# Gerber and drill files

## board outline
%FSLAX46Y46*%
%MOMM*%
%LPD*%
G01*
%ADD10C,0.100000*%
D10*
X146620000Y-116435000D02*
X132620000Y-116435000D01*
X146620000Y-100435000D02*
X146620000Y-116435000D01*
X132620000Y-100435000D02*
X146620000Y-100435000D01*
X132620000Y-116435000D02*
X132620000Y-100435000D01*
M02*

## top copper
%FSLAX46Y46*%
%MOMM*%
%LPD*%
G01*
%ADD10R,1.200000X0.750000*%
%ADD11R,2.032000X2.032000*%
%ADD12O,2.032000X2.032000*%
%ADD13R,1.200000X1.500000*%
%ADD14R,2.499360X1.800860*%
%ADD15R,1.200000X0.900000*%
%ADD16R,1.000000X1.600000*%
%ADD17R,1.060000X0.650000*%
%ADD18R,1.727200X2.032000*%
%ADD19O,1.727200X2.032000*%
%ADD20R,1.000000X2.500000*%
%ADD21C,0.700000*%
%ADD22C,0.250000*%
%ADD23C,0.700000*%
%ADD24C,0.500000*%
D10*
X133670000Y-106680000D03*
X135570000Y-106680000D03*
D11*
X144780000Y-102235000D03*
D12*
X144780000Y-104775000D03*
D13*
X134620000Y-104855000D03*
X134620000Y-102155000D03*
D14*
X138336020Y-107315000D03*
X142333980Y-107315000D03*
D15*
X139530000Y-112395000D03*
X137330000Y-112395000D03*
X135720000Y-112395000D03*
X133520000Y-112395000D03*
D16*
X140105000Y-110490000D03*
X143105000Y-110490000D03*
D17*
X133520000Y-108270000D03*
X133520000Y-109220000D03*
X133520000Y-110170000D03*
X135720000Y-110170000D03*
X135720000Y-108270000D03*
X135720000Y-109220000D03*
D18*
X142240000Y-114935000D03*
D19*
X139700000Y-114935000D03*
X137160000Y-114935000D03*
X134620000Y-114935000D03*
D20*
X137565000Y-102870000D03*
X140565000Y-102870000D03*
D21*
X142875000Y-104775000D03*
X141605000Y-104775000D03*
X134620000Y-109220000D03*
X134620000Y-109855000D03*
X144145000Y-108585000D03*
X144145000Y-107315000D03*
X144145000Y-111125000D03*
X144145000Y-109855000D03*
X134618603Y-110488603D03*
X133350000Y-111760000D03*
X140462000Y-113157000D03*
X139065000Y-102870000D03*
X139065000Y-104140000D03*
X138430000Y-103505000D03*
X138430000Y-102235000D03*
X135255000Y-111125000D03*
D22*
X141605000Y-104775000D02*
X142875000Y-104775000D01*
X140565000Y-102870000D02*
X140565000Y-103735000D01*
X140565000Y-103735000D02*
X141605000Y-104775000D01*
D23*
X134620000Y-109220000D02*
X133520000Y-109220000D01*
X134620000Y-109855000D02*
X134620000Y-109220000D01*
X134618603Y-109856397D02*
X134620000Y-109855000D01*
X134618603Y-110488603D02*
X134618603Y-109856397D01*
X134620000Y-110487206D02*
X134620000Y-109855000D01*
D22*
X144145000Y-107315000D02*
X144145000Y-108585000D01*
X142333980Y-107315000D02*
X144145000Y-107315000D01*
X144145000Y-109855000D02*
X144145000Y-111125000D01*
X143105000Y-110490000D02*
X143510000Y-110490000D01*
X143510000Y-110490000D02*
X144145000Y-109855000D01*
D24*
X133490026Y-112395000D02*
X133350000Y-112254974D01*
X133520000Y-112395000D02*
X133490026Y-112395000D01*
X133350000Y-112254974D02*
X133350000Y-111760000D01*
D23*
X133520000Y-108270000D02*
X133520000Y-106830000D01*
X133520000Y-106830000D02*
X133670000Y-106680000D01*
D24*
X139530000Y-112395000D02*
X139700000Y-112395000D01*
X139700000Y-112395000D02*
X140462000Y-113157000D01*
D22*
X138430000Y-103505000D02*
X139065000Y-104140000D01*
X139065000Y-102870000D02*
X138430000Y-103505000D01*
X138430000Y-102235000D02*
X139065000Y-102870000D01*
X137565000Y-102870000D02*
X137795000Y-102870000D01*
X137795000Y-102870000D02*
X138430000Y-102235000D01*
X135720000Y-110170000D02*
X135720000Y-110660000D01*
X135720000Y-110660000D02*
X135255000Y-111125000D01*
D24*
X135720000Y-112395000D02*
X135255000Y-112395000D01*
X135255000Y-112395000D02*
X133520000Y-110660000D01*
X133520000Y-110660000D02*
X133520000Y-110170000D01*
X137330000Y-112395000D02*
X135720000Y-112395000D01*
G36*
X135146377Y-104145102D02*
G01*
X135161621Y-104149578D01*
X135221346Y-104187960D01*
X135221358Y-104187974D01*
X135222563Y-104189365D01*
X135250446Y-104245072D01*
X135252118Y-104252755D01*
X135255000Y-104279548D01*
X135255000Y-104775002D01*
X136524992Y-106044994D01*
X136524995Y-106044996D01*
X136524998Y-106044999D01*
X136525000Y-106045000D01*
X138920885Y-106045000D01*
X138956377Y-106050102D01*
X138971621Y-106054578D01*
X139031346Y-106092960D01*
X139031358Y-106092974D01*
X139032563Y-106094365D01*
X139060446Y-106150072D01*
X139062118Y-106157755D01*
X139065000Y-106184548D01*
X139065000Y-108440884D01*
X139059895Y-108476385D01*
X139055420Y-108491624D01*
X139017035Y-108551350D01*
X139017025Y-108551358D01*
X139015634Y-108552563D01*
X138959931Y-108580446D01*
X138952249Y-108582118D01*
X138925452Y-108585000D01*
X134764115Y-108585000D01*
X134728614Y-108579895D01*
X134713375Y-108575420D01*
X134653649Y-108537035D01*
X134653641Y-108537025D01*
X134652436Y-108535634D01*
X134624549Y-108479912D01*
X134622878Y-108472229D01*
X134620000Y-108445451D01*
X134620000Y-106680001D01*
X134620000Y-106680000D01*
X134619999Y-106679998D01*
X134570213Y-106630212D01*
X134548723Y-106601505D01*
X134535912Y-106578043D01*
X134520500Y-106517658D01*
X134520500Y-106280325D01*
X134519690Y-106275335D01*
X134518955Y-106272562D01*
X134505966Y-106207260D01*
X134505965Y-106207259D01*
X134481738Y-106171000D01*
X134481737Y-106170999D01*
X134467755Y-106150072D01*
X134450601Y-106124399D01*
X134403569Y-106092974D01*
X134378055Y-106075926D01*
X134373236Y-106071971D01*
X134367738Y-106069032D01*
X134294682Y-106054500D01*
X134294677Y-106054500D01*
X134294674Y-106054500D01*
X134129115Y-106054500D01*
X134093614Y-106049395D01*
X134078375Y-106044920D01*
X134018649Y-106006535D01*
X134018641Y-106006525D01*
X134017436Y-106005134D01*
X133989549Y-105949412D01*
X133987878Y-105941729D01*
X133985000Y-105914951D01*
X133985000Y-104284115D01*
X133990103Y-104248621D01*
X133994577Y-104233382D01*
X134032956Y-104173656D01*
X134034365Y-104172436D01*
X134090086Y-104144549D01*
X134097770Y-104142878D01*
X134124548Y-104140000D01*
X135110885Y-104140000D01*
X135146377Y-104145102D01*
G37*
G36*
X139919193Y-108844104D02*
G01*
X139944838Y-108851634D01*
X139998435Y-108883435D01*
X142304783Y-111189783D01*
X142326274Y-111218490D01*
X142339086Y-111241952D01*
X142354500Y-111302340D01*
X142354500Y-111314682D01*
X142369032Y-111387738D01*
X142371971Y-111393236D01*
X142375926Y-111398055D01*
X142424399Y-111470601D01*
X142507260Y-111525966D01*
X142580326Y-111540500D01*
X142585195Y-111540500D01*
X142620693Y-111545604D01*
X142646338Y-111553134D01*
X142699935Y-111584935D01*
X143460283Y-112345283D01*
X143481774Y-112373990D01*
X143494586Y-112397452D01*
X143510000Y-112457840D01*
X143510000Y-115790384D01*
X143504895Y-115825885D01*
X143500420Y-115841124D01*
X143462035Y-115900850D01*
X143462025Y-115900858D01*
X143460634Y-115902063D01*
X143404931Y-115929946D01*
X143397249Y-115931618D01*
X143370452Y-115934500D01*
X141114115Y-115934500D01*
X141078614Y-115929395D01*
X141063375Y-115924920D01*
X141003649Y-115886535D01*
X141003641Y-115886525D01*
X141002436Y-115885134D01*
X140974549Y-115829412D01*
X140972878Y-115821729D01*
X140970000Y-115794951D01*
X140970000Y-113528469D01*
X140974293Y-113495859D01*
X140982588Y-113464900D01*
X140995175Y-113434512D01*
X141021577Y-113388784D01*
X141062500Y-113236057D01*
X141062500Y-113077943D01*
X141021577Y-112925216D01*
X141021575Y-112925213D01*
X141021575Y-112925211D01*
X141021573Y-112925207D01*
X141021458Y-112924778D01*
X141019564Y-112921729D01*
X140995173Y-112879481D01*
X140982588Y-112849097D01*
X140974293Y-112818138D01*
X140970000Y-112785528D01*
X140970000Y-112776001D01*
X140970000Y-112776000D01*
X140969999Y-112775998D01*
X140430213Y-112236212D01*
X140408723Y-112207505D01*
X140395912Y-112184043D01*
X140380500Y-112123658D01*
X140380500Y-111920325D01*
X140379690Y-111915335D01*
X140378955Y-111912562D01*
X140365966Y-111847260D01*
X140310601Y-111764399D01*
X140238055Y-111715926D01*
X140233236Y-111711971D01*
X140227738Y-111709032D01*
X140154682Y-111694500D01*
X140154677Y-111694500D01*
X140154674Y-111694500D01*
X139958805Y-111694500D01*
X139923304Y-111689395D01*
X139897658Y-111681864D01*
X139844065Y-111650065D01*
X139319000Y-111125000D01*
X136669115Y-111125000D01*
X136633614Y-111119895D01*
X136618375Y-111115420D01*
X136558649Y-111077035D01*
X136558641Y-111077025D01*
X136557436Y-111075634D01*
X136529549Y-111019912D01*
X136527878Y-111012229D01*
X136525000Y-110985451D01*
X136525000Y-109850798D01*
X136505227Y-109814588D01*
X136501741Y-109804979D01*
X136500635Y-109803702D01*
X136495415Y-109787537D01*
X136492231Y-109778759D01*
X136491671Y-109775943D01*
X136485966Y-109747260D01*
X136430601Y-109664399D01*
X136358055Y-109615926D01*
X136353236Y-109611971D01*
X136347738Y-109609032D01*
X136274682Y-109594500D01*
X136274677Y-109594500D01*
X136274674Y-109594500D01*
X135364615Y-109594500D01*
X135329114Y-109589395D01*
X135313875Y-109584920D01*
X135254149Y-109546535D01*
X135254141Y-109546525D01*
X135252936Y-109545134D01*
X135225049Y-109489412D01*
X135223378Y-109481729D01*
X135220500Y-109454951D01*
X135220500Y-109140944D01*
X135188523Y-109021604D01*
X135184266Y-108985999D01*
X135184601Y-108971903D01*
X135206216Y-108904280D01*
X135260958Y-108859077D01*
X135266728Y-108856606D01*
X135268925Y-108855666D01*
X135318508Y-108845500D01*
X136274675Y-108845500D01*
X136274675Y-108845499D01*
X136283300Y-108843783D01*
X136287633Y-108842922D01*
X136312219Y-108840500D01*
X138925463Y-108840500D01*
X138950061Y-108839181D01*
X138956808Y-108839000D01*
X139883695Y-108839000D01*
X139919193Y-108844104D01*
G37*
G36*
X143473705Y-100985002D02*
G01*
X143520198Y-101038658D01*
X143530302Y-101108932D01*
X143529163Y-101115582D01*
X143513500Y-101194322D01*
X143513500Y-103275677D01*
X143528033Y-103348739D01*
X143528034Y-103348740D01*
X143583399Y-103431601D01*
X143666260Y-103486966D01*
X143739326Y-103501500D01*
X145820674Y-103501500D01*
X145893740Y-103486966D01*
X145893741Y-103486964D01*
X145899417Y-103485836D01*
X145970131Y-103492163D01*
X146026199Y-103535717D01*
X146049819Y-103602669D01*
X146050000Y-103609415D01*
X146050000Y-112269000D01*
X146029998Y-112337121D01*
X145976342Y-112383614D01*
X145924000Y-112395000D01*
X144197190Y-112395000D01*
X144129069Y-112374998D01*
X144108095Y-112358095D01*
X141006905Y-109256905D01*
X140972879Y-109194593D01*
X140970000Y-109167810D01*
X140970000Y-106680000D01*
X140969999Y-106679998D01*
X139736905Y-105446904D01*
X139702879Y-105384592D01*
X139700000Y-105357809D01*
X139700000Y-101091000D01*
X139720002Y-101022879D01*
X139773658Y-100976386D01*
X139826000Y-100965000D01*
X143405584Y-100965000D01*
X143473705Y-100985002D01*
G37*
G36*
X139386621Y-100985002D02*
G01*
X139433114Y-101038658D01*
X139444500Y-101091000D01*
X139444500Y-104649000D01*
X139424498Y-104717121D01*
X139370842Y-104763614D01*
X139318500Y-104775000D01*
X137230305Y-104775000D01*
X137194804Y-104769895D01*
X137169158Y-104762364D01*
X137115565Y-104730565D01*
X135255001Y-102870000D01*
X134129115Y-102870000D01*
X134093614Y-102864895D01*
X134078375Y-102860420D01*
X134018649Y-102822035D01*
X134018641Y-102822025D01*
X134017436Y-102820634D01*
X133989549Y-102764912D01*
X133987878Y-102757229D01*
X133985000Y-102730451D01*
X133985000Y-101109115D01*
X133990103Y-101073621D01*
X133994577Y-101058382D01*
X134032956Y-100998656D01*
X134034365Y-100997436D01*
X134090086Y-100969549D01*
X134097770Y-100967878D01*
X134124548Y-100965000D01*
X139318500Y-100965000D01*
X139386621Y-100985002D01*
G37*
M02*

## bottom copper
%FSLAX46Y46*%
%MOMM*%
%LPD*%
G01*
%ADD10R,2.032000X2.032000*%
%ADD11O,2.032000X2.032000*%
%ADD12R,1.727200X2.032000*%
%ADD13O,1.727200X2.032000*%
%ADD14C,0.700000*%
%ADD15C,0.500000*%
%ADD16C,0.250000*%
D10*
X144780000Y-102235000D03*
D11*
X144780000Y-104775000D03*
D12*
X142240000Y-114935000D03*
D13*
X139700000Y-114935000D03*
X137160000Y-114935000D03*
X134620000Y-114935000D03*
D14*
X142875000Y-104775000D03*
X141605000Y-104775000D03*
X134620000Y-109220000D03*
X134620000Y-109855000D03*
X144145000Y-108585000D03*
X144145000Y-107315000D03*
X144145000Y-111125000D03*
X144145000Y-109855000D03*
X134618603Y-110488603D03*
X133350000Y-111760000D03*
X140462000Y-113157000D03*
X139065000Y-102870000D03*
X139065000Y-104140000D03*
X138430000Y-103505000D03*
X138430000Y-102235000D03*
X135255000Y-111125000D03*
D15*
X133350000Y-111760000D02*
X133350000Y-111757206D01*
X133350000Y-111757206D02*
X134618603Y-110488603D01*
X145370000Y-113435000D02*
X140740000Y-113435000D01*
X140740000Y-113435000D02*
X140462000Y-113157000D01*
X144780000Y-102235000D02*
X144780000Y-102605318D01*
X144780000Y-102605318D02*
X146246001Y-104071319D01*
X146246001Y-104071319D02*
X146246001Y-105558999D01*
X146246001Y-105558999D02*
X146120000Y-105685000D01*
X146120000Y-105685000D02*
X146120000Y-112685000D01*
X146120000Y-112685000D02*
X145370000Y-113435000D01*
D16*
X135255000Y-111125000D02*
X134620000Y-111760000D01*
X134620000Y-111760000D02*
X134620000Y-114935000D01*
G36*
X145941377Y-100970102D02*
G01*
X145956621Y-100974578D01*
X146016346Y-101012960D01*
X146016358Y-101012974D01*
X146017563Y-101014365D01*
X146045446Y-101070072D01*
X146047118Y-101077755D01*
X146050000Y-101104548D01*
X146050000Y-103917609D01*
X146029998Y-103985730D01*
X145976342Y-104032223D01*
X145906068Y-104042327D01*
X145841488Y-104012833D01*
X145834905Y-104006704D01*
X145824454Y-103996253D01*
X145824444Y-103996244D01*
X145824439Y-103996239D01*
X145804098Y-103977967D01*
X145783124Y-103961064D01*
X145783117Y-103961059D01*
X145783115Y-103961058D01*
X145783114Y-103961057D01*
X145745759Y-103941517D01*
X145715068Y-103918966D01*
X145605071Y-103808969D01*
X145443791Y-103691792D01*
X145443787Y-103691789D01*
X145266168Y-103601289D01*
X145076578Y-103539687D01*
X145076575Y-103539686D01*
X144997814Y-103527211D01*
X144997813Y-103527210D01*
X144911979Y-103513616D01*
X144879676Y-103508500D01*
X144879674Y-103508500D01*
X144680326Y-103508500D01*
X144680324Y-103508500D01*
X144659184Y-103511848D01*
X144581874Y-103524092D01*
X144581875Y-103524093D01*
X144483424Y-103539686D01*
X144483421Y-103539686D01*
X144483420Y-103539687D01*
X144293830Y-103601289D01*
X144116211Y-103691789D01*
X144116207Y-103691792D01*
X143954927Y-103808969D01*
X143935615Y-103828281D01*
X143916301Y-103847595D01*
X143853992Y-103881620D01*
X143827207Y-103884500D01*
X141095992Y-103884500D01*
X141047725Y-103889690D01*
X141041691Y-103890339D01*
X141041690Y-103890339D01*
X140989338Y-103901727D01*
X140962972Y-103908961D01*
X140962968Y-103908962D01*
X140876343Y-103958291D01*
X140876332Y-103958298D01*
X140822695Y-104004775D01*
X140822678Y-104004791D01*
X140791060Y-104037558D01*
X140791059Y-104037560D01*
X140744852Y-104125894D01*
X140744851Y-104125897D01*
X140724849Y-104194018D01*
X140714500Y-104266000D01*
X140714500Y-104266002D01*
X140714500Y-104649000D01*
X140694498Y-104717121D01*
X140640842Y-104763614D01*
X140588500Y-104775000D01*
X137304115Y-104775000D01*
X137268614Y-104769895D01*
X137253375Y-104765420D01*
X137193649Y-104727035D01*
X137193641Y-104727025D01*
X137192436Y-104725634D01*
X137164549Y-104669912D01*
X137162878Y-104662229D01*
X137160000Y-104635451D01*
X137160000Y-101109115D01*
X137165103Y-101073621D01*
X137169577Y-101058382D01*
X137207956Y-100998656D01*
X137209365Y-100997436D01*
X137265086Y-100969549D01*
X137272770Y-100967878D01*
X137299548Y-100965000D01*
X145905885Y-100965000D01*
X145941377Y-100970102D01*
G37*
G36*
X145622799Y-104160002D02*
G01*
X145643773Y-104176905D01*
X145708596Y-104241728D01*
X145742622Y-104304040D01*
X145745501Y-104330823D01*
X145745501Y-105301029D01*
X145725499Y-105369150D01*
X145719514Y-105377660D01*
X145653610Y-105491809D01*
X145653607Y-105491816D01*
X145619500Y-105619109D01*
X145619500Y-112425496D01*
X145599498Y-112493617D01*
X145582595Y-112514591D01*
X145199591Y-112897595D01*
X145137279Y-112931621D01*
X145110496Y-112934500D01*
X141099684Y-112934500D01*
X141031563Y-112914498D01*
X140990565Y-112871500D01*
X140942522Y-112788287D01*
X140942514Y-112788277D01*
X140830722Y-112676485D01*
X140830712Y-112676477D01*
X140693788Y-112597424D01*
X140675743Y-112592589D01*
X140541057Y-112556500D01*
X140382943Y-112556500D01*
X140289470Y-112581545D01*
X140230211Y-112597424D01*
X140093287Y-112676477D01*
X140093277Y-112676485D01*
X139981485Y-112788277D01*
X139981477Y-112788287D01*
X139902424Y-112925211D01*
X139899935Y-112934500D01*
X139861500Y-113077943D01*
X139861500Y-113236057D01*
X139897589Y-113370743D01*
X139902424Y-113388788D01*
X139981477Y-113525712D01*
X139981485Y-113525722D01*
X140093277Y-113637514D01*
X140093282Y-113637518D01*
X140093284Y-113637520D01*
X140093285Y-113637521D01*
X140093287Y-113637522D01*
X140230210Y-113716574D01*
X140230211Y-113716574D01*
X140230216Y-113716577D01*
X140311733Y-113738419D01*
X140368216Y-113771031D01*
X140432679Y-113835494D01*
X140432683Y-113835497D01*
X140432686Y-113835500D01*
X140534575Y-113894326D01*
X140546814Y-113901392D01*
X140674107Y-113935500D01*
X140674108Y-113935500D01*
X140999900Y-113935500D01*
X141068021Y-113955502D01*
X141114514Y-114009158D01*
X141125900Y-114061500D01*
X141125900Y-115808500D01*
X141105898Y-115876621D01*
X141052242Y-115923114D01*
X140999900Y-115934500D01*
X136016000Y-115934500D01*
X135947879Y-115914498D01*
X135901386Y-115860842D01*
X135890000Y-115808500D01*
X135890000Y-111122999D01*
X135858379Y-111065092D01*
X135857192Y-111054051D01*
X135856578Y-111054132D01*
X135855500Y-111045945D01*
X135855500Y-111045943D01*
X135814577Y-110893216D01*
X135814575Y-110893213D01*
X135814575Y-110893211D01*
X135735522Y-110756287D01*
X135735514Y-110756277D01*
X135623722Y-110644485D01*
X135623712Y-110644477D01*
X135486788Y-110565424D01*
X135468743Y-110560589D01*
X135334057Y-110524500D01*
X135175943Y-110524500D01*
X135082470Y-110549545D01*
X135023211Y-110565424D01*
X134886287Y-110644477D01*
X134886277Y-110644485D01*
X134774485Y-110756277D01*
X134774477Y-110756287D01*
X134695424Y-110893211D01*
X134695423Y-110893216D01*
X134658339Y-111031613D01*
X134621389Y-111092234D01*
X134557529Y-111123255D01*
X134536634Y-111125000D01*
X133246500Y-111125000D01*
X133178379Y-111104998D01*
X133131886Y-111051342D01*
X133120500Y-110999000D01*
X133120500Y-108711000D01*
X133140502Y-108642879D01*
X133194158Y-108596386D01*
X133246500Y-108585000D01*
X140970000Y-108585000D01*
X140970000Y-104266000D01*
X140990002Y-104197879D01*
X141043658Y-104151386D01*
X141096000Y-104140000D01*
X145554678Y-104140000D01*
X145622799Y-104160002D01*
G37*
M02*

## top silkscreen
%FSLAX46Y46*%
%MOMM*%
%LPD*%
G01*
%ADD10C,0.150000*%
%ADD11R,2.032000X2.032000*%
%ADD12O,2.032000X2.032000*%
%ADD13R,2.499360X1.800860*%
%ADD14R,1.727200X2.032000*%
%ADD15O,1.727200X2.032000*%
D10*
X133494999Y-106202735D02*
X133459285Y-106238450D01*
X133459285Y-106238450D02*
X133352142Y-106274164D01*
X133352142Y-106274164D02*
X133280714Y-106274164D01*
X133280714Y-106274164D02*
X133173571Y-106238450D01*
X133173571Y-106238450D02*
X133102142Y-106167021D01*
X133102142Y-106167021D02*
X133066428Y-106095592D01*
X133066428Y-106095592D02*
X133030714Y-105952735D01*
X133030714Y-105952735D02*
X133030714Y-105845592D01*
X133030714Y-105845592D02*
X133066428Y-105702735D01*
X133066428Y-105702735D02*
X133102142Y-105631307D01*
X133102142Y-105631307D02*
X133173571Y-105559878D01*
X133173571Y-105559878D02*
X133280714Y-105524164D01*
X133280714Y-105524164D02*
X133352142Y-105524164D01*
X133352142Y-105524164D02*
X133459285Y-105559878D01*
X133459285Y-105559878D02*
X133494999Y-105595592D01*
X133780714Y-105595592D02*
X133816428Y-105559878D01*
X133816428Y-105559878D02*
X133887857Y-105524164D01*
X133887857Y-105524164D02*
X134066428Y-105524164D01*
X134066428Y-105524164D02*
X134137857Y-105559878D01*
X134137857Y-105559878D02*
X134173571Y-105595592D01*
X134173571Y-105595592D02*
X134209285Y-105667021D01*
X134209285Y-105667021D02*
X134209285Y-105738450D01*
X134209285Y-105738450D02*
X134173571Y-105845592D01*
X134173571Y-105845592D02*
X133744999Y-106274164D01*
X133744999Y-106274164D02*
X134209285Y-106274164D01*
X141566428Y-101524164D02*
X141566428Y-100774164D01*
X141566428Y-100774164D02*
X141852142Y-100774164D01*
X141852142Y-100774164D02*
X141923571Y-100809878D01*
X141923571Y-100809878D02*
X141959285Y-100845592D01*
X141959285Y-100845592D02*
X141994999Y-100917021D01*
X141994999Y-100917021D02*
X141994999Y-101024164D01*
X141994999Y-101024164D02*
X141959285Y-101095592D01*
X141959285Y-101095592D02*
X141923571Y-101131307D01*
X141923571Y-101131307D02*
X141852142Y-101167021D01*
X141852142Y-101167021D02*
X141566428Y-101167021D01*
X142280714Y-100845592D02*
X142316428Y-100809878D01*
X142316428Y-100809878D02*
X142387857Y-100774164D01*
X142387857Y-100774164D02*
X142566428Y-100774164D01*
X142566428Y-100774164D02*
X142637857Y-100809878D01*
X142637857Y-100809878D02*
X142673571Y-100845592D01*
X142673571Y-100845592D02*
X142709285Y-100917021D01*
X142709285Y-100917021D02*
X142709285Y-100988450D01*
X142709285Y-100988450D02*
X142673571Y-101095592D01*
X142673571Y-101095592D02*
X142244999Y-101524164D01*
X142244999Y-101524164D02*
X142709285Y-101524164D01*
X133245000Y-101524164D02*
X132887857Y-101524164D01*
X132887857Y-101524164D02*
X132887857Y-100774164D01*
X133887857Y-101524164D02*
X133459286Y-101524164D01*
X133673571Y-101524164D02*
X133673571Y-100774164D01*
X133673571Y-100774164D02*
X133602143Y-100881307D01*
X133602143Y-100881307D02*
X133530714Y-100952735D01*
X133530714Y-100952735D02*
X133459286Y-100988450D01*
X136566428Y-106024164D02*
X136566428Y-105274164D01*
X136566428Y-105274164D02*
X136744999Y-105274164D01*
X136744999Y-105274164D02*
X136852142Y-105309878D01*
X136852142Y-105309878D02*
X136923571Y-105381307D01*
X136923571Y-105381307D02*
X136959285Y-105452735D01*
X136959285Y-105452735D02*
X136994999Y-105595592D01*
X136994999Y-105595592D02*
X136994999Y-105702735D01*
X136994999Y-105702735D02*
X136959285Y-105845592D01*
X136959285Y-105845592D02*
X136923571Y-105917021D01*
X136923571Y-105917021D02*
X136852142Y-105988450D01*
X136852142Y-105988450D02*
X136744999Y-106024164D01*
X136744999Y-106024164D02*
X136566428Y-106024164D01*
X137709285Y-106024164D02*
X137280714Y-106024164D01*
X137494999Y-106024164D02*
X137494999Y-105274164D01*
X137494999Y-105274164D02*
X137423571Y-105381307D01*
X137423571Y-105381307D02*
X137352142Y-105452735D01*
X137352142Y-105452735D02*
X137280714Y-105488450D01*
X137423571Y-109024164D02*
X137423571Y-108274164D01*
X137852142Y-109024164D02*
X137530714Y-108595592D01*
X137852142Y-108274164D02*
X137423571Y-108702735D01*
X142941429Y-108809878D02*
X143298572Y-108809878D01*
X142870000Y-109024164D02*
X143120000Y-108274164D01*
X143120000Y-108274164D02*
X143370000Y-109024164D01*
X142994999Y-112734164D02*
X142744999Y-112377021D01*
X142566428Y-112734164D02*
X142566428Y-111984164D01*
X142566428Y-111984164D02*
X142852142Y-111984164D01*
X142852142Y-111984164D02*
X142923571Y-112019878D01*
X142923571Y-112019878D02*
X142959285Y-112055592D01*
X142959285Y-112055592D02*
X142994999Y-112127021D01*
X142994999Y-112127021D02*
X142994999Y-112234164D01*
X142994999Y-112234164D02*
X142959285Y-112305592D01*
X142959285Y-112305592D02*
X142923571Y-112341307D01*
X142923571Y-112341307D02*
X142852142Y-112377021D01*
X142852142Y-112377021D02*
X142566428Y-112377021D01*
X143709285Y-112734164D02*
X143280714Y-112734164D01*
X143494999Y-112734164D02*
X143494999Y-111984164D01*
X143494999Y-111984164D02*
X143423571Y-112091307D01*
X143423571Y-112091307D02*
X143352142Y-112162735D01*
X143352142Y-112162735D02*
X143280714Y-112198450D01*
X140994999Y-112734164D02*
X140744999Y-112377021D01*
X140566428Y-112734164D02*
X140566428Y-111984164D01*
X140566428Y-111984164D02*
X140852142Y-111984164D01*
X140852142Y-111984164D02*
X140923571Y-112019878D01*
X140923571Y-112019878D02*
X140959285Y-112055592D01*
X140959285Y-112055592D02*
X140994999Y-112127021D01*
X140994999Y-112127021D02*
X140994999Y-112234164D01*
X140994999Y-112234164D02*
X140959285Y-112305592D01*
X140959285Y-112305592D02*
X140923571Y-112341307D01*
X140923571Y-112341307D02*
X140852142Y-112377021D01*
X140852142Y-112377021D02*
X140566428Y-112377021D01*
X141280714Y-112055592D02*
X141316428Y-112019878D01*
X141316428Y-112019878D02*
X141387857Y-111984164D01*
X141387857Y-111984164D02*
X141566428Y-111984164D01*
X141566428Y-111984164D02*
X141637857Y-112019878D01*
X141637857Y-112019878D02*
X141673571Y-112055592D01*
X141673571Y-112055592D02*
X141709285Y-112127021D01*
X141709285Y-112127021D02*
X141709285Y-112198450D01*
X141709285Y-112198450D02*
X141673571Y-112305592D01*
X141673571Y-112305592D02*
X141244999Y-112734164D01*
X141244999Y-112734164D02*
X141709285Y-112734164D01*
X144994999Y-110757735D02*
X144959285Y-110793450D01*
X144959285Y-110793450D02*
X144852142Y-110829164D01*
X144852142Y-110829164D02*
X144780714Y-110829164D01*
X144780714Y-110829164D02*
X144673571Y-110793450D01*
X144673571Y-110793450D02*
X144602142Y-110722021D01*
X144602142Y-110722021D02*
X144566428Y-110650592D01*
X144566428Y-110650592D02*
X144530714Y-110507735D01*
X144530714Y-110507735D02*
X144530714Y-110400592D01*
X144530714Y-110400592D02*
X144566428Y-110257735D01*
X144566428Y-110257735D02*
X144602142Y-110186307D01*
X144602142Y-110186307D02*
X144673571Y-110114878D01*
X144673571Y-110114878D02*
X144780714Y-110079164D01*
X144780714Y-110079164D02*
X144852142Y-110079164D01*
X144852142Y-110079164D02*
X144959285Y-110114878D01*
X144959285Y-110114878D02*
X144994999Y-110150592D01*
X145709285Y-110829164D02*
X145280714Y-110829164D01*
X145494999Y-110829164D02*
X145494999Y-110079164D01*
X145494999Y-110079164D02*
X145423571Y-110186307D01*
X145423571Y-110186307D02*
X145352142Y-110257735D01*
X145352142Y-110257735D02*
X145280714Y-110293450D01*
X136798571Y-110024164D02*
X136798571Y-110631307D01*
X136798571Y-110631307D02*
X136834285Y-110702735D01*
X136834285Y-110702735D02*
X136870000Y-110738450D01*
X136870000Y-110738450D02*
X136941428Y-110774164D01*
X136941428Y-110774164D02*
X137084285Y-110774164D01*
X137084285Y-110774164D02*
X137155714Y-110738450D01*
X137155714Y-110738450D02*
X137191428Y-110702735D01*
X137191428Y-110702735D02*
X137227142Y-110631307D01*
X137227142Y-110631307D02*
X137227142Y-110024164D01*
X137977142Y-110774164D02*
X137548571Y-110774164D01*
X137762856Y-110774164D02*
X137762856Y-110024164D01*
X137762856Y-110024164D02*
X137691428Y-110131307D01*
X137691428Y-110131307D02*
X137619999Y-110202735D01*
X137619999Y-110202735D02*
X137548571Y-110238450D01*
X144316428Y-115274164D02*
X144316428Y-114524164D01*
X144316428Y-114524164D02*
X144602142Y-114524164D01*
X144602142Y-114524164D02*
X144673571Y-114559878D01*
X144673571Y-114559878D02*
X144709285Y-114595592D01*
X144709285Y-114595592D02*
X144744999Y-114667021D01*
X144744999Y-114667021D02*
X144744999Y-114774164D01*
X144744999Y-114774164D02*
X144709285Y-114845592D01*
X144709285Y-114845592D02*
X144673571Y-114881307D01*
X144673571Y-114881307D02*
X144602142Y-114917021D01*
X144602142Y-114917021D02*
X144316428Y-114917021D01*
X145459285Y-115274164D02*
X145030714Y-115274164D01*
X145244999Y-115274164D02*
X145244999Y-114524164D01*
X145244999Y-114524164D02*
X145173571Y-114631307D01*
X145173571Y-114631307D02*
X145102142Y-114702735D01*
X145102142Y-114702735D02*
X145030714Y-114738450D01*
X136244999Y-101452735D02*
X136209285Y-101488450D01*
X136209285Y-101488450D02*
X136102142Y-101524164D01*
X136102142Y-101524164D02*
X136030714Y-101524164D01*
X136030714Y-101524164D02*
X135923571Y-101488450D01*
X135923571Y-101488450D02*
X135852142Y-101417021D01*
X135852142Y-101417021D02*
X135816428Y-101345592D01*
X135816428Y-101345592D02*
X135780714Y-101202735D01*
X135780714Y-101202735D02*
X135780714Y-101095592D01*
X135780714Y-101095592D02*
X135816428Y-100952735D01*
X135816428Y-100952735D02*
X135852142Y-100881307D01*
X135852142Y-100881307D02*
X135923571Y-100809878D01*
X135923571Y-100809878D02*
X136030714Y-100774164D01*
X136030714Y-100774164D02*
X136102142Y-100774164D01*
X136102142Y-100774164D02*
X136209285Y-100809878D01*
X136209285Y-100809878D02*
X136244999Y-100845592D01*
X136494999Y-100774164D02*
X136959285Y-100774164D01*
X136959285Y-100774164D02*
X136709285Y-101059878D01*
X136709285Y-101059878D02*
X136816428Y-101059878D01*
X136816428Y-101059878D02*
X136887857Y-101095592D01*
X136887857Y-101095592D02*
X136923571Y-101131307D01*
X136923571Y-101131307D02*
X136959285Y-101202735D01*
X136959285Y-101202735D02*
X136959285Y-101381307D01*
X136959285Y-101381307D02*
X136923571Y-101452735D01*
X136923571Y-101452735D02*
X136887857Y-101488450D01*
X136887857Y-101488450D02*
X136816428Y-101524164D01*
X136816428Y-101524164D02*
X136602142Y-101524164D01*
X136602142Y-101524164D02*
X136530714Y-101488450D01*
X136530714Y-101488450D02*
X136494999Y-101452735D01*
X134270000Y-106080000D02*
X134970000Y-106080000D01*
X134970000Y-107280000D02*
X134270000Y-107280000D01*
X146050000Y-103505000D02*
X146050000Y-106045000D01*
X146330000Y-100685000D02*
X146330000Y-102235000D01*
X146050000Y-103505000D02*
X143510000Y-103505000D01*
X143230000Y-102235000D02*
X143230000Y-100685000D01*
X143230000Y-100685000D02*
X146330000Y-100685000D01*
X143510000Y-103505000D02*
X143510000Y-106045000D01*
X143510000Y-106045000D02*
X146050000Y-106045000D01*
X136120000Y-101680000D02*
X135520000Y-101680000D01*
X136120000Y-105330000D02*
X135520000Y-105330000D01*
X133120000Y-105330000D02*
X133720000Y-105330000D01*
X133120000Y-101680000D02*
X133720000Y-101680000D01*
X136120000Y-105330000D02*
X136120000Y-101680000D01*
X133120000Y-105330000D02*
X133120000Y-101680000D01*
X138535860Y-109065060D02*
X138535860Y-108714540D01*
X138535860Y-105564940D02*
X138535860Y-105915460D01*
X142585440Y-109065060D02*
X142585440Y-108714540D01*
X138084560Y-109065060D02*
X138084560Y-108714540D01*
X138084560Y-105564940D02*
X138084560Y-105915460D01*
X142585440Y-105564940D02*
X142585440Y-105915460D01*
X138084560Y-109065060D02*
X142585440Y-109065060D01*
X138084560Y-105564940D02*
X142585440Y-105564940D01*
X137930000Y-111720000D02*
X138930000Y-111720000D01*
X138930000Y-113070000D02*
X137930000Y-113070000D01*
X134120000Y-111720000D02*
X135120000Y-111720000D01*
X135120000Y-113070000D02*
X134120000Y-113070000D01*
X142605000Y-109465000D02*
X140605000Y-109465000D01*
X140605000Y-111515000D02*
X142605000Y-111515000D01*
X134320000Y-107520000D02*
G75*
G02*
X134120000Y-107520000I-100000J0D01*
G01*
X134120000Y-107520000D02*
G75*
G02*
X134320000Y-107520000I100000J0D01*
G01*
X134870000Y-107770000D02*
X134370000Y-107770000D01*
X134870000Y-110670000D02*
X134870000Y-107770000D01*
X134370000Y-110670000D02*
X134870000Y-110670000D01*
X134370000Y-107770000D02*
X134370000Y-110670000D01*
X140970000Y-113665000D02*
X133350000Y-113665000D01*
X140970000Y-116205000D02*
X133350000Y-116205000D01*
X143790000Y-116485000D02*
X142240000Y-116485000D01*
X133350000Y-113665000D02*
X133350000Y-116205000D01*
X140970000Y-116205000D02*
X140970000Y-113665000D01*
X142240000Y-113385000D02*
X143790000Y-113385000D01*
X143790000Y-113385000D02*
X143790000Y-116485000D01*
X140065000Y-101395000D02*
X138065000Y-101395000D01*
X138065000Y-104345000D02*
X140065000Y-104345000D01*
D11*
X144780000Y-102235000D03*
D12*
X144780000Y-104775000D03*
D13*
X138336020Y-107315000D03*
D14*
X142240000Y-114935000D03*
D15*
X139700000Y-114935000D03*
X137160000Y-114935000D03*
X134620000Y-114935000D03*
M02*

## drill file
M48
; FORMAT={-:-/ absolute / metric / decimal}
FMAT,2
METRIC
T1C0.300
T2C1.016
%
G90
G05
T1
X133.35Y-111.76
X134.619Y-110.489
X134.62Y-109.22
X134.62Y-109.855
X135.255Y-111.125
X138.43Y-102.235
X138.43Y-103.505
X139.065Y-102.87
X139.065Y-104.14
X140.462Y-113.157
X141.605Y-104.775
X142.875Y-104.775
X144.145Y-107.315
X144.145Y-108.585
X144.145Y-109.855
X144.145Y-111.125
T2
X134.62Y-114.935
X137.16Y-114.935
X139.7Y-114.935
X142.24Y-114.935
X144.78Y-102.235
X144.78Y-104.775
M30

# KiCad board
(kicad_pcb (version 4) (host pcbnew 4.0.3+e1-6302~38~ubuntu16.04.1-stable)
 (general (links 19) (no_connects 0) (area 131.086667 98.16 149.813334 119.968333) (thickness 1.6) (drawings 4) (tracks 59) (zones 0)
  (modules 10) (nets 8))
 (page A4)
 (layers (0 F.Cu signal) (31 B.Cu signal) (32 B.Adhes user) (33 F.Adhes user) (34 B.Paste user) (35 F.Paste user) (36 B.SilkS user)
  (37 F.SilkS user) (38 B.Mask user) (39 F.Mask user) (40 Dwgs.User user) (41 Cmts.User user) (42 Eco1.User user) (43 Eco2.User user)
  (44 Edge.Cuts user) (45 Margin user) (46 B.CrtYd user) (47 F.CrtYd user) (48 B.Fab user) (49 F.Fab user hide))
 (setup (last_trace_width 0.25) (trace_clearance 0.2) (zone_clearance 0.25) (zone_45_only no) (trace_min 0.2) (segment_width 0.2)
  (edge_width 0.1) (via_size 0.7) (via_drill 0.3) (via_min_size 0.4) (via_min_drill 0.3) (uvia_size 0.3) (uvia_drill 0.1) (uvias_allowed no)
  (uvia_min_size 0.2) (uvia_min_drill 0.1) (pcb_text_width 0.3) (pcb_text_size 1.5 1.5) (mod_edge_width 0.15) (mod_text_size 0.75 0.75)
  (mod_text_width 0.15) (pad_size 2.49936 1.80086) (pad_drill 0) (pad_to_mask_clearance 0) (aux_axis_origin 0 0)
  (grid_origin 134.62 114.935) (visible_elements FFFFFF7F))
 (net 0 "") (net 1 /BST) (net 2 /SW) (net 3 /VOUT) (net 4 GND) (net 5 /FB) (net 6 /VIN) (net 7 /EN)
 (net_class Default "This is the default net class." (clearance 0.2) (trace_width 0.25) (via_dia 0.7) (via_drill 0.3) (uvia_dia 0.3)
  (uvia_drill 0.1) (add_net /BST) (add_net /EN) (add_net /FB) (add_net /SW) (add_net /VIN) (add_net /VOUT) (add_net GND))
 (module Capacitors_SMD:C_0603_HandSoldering (layer F.Cu) (at 134.62 106.68)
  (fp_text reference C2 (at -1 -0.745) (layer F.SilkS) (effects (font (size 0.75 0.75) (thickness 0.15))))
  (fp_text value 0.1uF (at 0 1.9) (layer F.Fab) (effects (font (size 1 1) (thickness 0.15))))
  (fp_line (start -0.35 -0.6) (end 0.35 -0.6) (layer F.SilkS) (width 0.15))
  (fp_line (start 0.35 0.6) (end -0.35 0.6) (layer F.SilkS) (width 0.15))
  (pad 1 smd rect (at -0.95 0) (size 1.2 0.75) (layers F.Cu F.Paste F.Mask) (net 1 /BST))
  (pad 2 smd rect (at 0.95 0) (size 1.2 0.75) (layers F.Cu F.Paste F.Mask) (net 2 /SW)))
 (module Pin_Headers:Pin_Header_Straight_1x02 (layer F.Cu) (at 144.78 102.235)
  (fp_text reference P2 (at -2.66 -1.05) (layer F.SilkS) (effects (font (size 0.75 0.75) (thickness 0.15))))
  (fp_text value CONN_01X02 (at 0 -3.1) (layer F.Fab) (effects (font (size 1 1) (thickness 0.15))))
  (fp_line (start 1.27 1.27) (end 1.27 3.81) (layer F.SilkS) (width 0.15))
  (fp_line (start 1.55 -1.55) (end 1.55 0) (layer F.SilkS) (width 0.15))
  (fp_line (start 1.27 1.27) (end -1.27 1.27) (layer F.SilkS) (width 0.15))
  (fp_line (start -1.55 0) (end -1.55 -1.55) (layer F.SilkS) (width 0.15))
  (fp_line (start -1.55 -1.55) (end 1.55 -1.55) (layer F.SilkS) (width 0.15))
  (fp_line (start -1.27 1.27) (end -1.27 3.81) (layer F.SilkS) (width 0.15))
  (fp_line (start -1.27 3.81) (end 1.27 3.81) (layer F.SilkS) (width 0.15))
  (pad 1 thru_hole rect (at 0 0) (size 2.032 2.032) (drill 1.016) (layers *.Cu *.Mask F.SilkS) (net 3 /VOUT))
  (pad 2 thru_hole oval (at 0 2.54) (size 2.032 2.032) (drill 1.016) (layers *.Cu *.Mask F.SilkS) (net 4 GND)))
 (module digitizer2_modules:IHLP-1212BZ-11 (layer F.Cu) (at 134.62 103.505 90)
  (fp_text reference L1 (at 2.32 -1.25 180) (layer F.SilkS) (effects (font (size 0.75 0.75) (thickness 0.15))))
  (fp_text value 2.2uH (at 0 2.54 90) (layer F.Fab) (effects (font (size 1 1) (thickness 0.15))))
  (fp_line (start 1.825 1.5) (end 1.825 0.9) (layer F.SilkS) (width 0.15))
  (fp_line (start -1.825 1.5) (end -1.825 0.9) (layer F.SilkS) (width 0.15))
  (fp_line (start -1.825 -1.5) (end -1.825 -0.9) (layer F.SilkS) (width 0.15))
  (fp_line (start 1.825 -1.5) (end 1.825 -0.9) (layer F.SilkS) (width 0.15))
  (fp_line (start -1.825 1.5) (end 1.825 1.5) (layer F.SilkS) (width 0.15))
  (fp_line (start -1.825 -1.5) (end 1.825 -1.5) (layer F.SilkS) (width 0.15))
  (pad 1 smd rect (at -1.35 0 90) (size 1.5 1.2) (layers F.Cu F.Paste F.Mask) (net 2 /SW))
  (pad 2 smd rect (at 1.35 0 90) (size 1.5 1.2) (layers F.Cu F.Paste F.Mask) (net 3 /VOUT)))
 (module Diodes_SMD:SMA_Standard (layer F.Cu) (at 140.335 107.315)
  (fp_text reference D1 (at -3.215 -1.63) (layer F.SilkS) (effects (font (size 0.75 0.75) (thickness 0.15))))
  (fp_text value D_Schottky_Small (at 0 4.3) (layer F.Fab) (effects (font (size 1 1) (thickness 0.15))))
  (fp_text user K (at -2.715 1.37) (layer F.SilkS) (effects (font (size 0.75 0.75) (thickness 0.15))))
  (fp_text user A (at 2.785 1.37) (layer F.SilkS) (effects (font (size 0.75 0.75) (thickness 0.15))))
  (fp_line (start -1.79914 1.75006) (end -1.79914 1.39954) (layer F.SilkS) (width 0.15))
  (fp_line (start -1.79914 -1.75006) (end -1.79914 -1.39954) (layer F.SilkS) (width 0.15))
  (fp_line (start 2.25044 1.75006) (end 2.25044 1.39954) (layer F.SilkS) (width 0.15))
  (fp_line (start -2.25044 1.75006) (end -2.25044 1.39954) (layer F.SilkS) (width 0.15))
  (fp_line (start -2.25044 -1.75006) (end -2.25044 -1.39954) (layer F.SilkS) (width 0.15))
  (fp_line (start 2.25044 -1.75006) (end 2.25044 -1.39954) (layer F.SilkS) (width 0.15))
  (fp_line (start -2.25044 1.75006) (end 2.25044 1.75006) (layer F.SilkS) (width 0.15))
  (fp_line (start -2.25044 -1.75006) (end 2.25044 -1.75006) (layer F.SilkS) (width 0.15))
  (pad 1 smd rect (at -1.99898 0) (size 2.49936 1.80086) (layers F.Cu F.Paste F.SilkS F.Mask) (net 2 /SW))
  (pad 2 smd rect (at 1.99898 0) (size 2.49936 1.80086) (layers F.Cu F.Paste F.Mask) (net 4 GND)))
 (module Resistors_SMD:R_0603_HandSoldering (layer F.Cu) (at 138.43 112.395 180)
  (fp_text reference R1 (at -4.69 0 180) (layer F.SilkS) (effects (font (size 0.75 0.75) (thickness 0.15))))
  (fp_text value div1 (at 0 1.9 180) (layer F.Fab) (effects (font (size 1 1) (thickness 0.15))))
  (fp_line (start 0.5 0.675) (end -0.5 0.675) (layer F.SilkS) (width 0.15))
  (fp_line (start -0.5 -0.675) (end 0.5 -0.675) (layer F.SilkS) (width 0.15))
  (pad 1 smd rect (at -1.1 0 180) (size 1.2 0.9) (layers F.Cu F.Paste F.Mask) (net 3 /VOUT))
  (pad 2 smd rect (at 1.1 0 180) (size 1.2 0.9) (layers F.Cu F.Paste F.Mask) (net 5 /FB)))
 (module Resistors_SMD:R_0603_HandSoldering (layer F.Cu) (at 134.62 112.395 180)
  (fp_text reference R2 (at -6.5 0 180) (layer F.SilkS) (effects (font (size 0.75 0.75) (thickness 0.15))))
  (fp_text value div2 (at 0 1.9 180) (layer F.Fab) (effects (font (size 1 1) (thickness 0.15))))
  (fp_line (start 0.5 0.675) (end -0.5 0.675) (layer F.SilkS) (width 0.15))
  (fp_line (start -0.5 -0.675) (end 0.5 -0.675) (layer F.SilkS) (width 0.15))
  (pad 1 smd rect (at -1.1 0 180) (size 1.2 0.9) (layers F.Cu F.Paste F.Mask) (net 5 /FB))
  (pad 2 smd rect (at 1.1 0 180) (size 1.2 0.9) (layers F.Cu F.Paste F.Mask) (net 4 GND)))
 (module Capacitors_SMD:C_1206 (layer F.Cu) (at 141.605 110.49)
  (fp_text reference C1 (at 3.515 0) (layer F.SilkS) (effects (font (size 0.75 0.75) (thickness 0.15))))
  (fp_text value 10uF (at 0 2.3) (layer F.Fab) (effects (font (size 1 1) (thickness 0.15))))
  (fp_line (start 1 -1.025) (end -1 -1.025) (layer F.SilkS) (width 0.15))
  (fp_line (start -1 1.025) (end 1 1.025) (layer F.SilkS) (width 0.15))
  (pad 1 smd rect (at -1.5 0) (size 1 1.6) (layers F.Cu F.Paste F.Mask) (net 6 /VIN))
  (pad 2 smd rect (at 1.5 0) (size 1 1.6) (layers F.Cu F.Paste F.Mask) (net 4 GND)))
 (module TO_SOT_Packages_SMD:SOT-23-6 (layer F.Cu) (at 134.62 109.22)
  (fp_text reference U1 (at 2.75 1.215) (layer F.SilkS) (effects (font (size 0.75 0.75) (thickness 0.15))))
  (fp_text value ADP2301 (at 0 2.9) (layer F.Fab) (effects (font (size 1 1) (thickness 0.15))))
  (fp_circle (center -0.4 -1.7) (end -0.3 -1.7) (layer F.SilkS) (width 0.15))
  (fp_line (start 0.25 -1.45) (end -0.25 -1.45) (layer F.SilkS) (width 0.15))
  (fp_line (start 0.25 1.45) (end 0.25 -1.45) (layer F.SilkS) (width 0.15))
  (fp_line (start -0.25 1.45) (end 0.25 1.45) (layer F.SilkS) (width 0.15))
  (fp_line (start -0.25 -1.45) (end -0.25 1.45) (layer F.SilkS) (width 0.15))
  (pad 1 smd rect (at -1.1 -0.95) (size 1.06 0.65) (layers F.Cu F.Paste F.Mask) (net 1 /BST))
  (pad 2 smd rect (at -1.1 0) (size 1.06 0.65) (layers F.Cu F.Paste F.Mask) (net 4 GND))
  (pad 3 smd rect (at -1.1 0.95) (size 1.06 0.65) (layers F.Cu F.Paste F.Mask) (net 5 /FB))
  (pad 4 smd rect (at 1.1 0.95) (size 1.06 0.65) (layers F.Cu F.Paste F.Mask) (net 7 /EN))
  (pad 6 smd rect (at 1.1 -0.95) (size 1.06 0.65) (layers F.Cu F.Paste F.Mask) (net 2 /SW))
  (pad 5 smd rect (at 1.1 0) (size 1.06 0.65) (layers F.Cu F.Paste F.Mask) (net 6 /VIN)))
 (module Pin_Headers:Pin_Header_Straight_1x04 (layer F.Cu) (at 142.24 114.935 270)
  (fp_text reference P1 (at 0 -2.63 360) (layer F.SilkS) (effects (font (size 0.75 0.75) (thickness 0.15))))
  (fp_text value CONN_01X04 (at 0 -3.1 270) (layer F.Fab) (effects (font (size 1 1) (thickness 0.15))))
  (fp_line (start -1.27 1.27) (end -1.27 8.89) (layer F.SilkS) (width 0.15))
  (fp_line (start 1.27 1.27) (end 1.27 8.89) (layer F.SilkS) (width 0.15))
  (fp_line (start 1.55 -1.55) (end 1.55 0) (layer F.SilkS) (width 0.15))
  (fp_line (start -1.27 8.89) (end 1.27 8.89) (layer F.SilkS) (width 0.15))
  (fp_line (start 1.27 1.27) (end -1.27 1.27) (layer F.SilkS) (width 0.15))
  (fp_line (start -1.55 0) (end -1.55 -1.55) (layer F.SilkS) (width 0.15))
  (fp_line (start -1.55 -1.55) (end 1.55 -1.55) (layer F.SilkS) (width 0.15))
  (pad 1 thru_hole rect (at 0 0 270) (size 2.032 1.7272) (drill 1.016) (layers *.Cu *.Mask F.SilkS) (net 6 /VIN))
  (pad 2 thru_hole oval (at 0 2.54 270) (size 2.032 1.7272) (drill 1.016) (layers *.Cu *.Mask F.SilkS) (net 4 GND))
  (pad 3 thru_hole oval (at 0 5.08 270) (size 2.032 1.7272) (drill 1.016) (layers *.Cu *.Mask F.SilkS) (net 4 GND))
  (pad 4 thru_hole oval (at 0 7.62 270) (size 2.032 1.7272) (drill 1.016) (layers *.Cu *.Mask F.SilkS) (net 7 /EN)))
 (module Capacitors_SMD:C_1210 (layer F.Cu) (at 139.065 102.87)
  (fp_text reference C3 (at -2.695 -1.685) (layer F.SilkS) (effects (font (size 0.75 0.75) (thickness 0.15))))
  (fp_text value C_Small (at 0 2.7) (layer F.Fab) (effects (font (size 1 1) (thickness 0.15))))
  (fp_line (start 1 -1.475) (end -1 -1.475) (layer F.SilkS) (width 0.15))
  (fp_line (start -1 1.475) (end 1 1.475) (layer F.SilkS) (width 0.15))
  (pad 1 smd rect (at -1.5 0) (size 1 2.5) (layers F.Cu F.Paste F.Mask) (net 3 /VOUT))
  (pad 2 smd rect (at 1.5 0) (size 1 2.5) (layers F.Cu F.Paste F.Mask) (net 4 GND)))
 (gr_line (start 146.62 116.435) (end 132.62 116.435) (layer Edge.Cuts) (width 0.1))
 (gr_line (start 146.62 100.435) (end 146.62 116.435) (layer Edge.Cuts) (width 0.1))
 (gr_line (start 132.62 100.435) (end 146.62 100.435) (layer Edge.Cuts) (width 0.1))
 (gr_line (start 132.62 116.435) (end 132.62 100.435) (layer Edge.Cuts) (width 0.1))
 (segment (start 141.605 104.775) (end 142.875 104.775) (width 0.25) (layer F.Cu) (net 4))
 (via (at 142.875 104.775) (size 0.7) (drill 0.3) (layers F.Cu B.Cu) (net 4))
 (segment (start 140.565 102.87) (end 140.565 103.735) (width 0.25) (layer F.Cu) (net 4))
 (segment (start 140.565 103.735) (end 141.605 104.775) (width 0.25) (layer F.Cu) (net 4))
 (via (at 141.605 104.775) (size 0.7) (drill 0.3) (layers F.Cu B.Cu) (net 4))
 (segment (start 134.62 109.22) (end 133.52 109.22) (width 0.7) (layer F.Cu) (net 4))
 (segment (start 134.62 109.855) (end 134.62 109.22) (width 0.7) (layer F.Cu) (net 4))
 (via (at 134.62 109.22) (size 0.7) (drill 0.3) (layers F.Cu B.Cu) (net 4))
 (segment (start 134.618603 109.856397) (end 134.62 109.855) (width 0.7) (layer F.Cu) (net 4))
 (segment (start 134.618603 110.488603) (end 134.618603 109.856397) (width 0.7) (layer F.Cu) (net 4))
 (segment (start 134.62 110.487206) (end 134.62 109.855) (width 0.7) (layer F.Cu) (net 4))
 (via (at 134.62 109.855) (size 0.7) (drill 0.3) (layers F.Cu B.Cu) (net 4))
 (segment (start 144.145 107.315) (end 144.145 108.585) (width 0.25) (layer F.Cu) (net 4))
 (via (at 144.145 108.585) (size 0.7) (drill 0.3) (layers F.Cu B.Cu) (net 4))
 (segment (start 142.33398 107.315) (end 144.145 107.315) (width 0.25) (layer F.Cu) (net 4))
 (via (at 144.145 107.315) (size 0.7) (drill 0.3) (layers F.Cu B.Cu) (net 4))
 (segment (start 144.145 109.855) (end 144.145 111.125) (width 0.25) (layer F.Cu) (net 4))
 (via (at 144.145 111.125) (size 0.7) (drill 0.3) (layers F.Cu B.Cu) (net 4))
 (segment (start 143.105 110.49) (end 143.51 110.49) (width 0.25) (layer F.Cu) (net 4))
 (segment (start 143.51 110.49) (end 144.145 109.855) (width 0.25) (layer F.Cu) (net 4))
 (via (at 144.145 109.855) (size 0.7) (drill 0.3) (layers F.Cu B.Cu) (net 4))
 (segment (start 133.35 111.76) (end 133.35 111.757206) (width 0.5) (layer B.Cu) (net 4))
 (segment (start 133.35 111.757206) (end 134.618603 110.488603) (width 0.5) (layer B.Cu) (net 4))
 (via (at 134.618603 110.488603) (size 0.7) (drill 0.3) (layers F.Cu B.Cu) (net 4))
 (segment (start 133.490026 112.395) (end 133.35 112.254974) (width 0.5) (layer F.Cu) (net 4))
 (segment (start 133.52 112.395) (end 133.490026 112.395) (width 0.5) (layer F.Cu) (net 4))
 (segment (start 133.35 112.254974) (end 133.35 111.76) (width 0.5) (layer F.Cu) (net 4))
 (via (at 133.35 111.76) (size 0.7) (drill 0.3) (layers F.Cu B.Cu) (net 4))
 (segment (start 133.52 108.27) (end 133.52 106.83) (width 0.7) (layer F.Cu) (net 1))
 (segment (start 133.52 106.83) (end 133.67 106.68) (width 0.7) (layer F.Cu) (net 1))
 (segment (start 139.53 112.395) (end 139.7 112.395) (width 0.5) (layer F.Cu) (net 3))
 (segment (start 139.7 112.395) (end 140.462 113.157) (width 0.5) (layer F.Cu) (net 3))
 (segment (start 145.37 113.435) (end 140.74 113.435) (width 0.5) (layer B.Cu) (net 3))
 (segment (start 140.74 113.435) (end 140.462 113.157) (width 0.5) (layer B.Cu) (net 3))
 (via (at 140.462 113.157) (size 0.7) (drill 0.3) (layers F.Cu B.Cu) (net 3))
 (segment (start 144.78 102.235) (end 144.78 102.605318) (width 0.5) (layer B.Cu) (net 3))
 (segment (start 144.78 102.605318) (end 146.246001 104.071319) (width 0.5) (layer B.Cu) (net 3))
 (segment (start 146.246001 104.071319) (end 146.246001 105.558999) (width 0.5) (layer B.Cu) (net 3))
 (segment (start 146.246001 105.558999) (end 146.12 105.685) (width 0.5) (layer B.Cu) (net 3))
 (segment (start 146.12 105.685) (end 146.12 112.685) (width 0.5) (layer B.Cu) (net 3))
 (segment (start 146.12 112.685) (end 145.37 113.435) (width 0.5) (layer B.Cu) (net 3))
 (via (at 139.065 102.87) (size 0.7) (drill 0.3) (layers F.Cu B.Cu) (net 3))
 (segment (start 138.43 103.505) (end 139.065 104.14) (width 0.25) (layer F.Cu) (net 3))
 (via (at 139.065 104.14) (size 0.7) (drill 0.3) (layers F.Cu B.Cu) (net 3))
 (segment (start 139.065 102.87) (end 138.43 103.505) (width 0.25) (layer F.Cu) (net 3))
 (via (at 138.43 103.505) (size 0.7) (drill 0.3) (layers F.Cu B.Cu) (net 3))
 (segment (start 138.43 102.235) (end 139.065 102.87) (width 0.25) (layer F.Cu) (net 3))
 (segment (start 137.565 102.87) (end 137.795 102.87) (width 0.25) (layer F.Cu) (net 3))
 (segment (start 137.795 102.87) (end 138.43 102.235) (width 0.25) (layer F.Cu) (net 3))
 (via (at 138.43 102.235) (size 0.7) (drill 0.3) (layers F.Cu B.Cu) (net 3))
 (segment (start 135.255 111.125) (end 134.62 111.76) (width 0.25) (layer B.Cu) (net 7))
 (segment (start 134.62 111.76) (end 134.62 114.935) (width 0.25) (layer B.Cu) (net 7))
 (segment (start 135.72 110.17) (end 135.72 110.66) (width 0.25) (layer F.Cu) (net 7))
 (segment (start 135.72 110.66) (end 135.255 111.125) (width 0.25) (layer F.Cu) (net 7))
 (via (at 135.255 111.125) (size 0.7) (drill 0.3) (layers F.Cu B.Cu) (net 7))
 (segment (start 135.72 112.395) (end 135.255 112.395) (width 0.5) (layer F.Cu) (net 5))
 (segment (start 135.255 112.395) (end 133.52 110.66) (width 0.5) (layer F.Cu) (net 5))
 (segment (start 133.52 110.66) (end 133.52 110.17) (width 0.5) (layer F.Cu) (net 5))
 (segment (start 137.33 112.395) (end 135.72 112.395) (width 0.5) (layer F.Cu) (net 5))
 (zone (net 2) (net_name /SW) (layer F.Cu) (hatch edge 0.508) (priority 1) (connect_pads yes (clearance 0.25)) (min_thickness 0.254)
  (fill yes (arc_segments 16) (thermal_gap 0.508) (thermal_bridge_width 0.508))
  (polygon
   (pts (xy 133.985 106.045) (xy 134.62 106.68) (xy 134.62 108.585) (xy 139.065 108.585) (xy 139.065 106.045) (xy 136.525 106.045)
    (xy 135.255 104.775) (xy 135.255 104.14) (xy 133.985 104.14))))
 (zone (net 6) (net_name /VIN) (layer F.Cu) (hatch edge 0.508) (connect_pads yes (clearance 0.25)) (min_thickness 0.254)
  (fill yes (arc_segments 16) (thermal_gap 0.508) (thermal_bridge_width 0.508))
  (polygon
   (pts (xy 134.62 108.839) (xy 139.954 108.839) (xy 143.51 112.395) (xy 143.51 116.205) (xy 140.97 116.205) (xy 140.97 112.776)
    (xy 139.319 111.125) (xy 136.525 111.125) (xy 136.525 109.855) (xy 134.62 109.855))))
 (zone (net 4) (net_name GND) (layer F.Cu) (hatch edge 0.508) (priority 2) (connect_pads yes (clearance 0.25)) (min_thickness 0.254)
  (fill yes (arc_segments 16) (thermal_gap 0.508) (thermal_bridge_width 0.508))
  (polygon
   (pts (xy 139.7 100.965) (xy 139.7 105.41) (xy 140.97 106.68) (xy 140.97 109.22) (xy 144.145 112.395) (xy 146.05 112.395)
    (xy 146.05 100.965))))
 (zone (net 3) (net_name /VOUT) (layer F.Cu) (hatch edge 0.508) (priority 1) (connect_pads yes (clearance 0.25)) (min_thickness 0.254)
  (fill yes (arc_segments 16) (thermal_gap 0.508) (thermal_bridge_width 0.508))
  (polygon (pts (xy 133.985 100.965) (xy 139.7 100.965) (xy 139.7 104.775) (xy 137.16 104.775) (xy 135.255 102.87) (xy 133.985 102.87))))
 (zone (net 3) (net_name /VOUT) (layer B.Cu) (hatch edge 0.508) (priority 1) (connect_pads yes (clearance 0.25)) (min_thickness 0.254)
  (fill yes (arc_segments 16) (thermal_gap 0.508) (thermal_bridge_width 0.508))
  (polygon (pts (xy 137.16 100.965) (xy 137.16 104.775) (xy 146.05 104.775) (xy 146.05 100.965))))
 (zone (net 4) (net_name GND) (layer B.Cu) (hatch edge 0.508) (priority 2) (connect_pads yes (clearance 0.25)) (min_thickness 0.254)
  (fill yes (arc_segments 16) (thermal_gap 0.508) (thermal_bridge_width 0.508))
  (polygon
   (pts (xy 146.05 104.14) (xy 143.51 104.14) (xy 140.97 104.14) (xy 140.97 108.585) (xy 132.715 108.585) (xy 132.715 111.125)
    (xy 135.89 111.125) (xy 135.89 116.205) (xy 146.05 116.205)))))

